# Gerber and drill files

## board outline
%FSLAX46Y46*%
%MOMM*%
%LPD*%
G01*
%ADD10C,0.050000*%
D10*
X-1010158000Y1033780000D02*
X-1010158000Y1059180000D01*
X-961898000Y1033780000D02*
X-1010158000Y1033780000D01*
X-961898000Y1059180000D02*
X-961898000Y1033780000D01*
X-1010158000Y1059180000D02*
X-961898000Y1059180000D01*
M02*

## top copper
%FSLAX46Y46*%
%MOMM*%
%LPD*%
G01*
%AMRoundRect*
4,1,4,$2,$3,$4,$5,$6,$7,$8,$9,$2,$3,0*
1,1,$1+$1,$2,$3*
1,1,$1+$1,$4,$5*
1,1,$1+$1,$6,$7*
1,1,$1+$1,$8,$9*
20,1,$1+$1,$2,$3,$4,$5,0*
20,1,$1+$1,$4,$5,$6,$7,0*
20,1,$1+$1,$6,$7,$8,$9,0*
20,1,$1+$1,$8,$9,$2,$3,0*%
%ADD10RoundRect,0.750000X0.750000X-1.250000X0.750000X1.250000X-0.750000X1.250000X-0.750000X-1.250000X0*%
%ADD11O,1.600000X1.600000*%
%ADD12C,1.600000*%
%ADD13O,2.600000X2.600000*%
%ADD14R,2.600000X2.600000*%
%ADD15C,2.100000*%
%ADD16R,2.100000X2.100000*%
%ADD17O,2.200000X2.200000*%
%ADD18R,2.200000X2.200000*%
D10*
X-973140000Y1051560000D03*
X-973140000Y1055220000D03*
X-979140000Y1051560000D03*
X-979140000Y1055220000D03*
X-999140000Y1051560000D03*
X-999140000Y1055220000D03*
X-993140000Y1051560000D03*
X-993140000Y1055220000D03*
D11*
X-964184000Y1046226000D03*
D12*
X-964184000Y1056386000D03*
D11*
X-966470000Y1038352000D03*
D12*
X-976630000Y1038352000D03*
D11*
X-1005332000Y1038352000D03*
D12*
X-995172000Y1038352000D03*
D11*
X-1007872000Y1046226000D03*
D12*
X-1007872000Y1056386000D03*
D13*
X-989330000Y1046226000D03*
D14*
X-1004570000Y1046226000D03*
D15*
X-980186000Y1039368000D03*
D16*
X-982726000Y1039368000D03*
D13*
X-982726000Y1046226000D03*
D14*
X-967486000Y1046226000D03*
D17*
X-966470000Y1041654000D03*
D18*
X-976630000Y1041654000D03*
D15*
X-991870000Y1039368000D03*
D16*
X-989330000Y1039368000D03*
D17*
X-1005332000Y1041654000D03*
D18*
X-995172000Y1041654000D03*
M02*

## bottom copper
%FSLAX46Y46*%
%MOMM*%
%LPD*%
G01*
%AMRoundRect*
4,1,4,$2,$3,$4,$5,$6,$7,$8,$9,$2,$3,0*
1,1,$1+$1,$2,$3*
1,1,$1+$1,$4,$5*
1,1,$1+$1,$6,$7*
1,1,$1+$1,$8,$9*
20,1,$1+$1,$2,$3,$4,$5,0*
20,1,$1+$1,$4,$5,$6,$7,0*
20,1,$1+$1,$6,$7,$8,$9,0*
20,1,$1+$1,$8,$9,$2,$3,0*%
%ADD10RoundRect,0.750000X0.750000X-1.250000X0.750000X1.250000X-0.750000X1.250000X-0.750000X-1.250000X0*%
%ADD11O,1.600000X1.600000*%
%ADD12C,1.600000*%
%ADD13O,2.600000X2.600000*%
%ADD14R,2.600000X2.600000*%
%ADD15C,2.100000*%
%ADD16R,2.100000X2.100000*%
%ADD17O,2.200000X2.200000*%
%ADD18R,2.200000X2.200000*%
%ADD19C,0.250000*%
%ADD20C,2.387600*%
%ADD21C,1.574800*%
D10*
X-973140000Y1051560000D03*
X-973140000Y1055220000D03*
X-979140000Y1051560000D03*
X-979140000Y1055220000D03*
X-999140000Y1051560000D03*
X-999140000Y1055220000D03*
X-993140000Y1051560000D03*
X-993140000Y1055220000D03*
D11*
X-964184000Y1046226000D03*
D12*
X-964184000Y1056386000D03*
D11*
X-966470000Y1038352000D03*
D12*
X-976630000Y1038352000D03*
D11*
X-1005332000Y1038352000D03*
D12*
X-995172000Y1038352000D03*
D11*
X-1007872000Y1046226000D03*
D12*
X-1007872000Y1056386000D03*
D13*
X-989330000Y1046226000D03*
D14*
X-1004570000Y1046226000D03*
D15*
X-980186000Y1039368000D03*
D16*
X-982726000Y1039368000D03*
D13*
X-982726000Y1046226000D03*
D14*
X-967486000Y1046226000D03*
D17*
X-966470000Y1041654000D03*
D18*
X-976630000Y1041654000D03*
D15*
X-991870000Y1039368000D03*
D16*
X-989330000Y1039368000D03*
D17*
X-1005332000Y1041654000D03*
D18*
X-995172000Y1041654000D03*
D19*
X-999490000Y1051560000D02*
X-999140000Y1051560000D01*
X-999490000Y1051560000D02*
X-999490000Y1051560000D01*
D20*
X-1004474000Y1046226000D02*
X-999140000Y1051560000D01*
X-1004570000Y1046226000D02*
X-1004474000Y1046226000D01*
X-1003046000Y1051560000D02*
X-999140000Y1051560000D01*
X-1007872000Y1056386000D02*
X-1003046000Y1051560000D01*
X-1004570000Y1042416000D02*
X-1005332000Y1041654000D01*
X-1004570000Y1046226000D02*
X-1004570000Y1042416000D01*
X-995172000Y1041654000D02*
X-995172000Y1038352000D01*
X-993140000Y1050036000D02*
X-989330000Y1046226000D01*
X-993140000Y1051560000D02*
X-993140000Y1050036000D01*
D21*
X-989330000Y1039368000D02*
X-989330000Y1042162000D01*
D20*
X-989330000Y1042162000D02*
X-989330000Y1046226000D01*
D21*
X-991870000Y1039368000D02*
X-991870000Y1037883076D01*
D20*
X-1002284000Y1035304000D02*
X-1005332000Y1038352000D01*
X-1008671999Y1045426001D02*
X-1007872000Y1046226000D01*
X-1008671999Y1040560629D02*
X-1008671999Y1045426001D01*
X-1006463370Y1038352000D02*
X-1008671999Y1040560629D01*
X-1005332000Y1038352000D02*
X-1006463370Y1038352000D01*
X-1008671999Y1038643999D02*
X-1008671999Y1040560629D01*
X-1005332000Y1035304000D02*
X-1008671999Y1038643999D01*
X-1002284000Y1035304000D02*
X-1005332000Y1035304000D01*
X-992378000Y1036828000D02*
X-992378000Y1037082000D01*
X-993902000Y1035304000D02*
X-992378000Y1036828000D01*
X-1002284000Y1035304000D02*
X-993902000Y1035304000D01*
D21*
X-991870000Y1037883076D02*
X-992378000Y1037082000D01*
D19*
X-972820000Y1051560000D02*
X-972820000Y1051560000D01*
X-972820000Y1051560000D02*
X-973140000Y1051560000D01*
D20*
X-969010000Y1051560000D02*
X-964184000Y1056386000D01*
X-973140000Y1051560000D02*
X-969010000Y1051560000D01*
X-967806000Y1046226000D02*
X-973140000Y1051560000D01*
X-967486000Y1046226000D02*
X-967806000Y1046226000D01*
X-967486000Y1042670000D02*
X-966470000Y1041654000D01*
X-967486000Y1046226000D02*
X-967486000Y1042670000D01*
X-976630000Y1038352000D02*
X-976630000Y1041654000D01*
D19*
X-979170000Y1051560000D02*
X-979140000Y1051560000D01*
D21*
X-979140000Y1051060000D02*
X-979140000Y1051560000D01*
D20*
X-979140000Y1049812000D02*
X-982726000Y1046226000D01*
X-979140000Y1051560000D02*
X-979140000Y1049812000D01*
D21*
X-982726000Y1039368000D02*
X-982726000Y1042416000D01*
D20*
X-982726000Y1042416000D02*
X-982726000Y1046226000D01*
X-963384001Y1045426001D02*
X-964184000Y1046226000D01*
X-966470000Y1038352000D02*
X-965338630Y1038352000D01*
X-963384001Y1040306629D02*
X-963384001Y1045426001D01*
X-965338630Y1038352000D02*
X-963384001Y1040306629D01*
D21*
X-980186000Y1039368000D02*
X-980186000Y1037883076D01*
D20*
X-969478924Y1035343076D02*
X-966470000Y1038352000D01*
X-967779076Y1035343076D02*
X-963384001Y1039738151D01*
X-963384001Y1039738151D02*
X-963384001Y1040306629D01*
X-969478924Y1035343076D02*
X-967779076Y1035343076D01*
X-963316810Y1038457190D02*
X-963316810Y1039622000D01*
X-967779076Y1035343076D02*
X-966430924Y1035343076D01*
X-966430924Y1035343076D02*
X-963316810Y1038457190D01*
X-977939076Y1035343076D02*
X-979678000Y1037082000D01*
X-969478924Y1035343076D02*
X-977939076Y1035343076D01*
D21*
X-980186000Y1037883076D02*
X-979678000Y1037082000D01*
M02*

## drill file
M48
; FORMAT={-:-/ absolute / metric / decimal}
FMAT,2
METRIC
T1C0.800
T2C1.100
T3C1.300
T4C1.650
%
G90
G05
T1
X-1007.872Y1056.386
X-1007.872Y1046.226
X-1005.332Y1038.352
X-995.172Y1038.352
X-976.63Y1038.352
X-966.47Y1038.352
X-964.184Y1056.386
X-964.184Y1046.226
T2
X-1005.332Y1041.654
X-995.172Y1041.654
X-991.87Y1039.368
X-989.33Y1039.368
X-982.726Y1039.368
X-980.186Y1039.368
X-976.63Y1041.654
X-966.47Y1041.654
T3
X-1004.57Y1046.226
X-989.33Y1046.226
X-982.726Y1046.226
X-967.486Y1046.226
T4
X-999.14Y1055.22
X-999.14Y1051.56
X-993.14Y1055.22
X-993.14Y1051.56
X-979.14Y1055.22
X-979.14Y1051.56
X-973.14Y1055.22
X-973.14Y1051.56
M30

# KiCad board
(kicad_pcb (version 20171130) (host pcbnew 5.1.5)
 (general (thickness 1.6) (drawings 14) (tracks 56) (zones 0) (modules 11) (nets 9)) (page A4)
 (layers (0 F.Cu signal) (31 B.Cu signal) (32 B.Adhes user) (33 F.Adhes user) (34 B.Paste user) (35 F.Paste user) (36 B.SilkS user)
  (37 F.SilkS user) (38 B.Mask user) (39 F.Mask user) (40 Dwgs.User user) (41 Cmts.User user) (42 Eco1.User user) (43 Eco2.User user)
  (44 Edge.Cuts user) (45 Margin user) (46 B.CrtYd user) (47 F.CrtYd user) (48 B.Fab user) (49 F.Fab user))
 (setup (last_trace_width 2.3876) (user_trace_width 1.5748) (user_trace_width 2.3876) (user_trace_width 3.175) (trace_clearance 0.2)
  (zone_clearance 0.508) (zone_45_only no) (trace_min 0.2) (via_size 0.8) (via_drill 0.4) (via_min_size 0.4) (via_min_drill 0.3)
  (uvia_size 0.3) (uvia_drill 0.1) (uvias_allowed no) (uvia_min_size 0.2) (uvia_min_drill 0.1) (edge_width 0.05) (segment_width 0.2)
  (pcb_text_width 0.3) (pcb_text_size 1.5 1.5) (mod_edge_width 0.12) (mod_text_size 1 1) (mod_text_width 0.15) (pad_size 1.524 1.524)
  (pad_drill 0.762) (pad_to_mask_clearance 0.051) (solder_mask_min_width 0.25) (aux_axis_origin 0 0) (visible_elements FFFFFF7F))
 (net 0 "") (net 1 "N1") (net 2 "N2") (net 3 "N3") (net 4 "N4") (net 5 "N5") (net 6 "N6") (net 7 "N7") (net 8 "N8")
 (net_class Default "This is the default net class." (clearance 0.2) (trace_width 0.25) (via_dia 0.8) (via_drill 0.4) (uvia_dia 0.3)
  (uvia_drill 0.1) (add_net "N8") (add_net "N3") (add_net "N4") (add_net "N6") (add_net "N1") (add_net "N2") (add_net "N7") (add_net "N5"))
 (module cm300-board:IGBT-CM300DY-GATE (layer F.Cu) (at -1000.64 -1049.56)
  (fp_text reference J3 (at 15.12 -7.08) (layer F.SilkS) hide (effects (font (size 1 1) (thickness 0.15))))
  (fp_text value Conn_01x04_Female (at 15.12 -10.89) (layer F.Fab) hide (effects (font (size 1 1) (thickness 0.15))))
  (pad 4 thru_hole roundrect (at 27.5 -2 90) (size 4 3) (drill 1.65) (layers *.Cu *.Mask) (roundrect_rratio 0.25) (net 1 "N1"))
  (pad 4 thru_hole roundrect (at 27.5 -5.66 90) (size 4 3) (drill 1.65) (layers *.Cu *.Mask) (roundrect_rratio 0.25) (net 1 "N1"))
  (pad 3 thru_hole roundrect (at 21.5 -2 90) (size 4 3) (drill 1.65) (layers *.Cu *.Mask) (roundrect_rratio 0.25) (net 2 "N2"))
  (pad 3 thru_hole roundrect (at 21.5 -5.66 90) (size 4 3) (drill 1.65) (layers *.Cu *.Mask) (roundrect_rratio 0.25) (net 2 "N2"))
  (pad 1 thru_hole roundrect (at 1.5 -2 90) (size 4 3) (drill 1.65) (layers *.Cu *.Mask) (roundrect_rratio 0.25) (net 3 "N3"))
  (pad 1 thru_hole roundrect (at 1.5 -5.66 90) (size 4 3) (drill 1.65) (layers *.Cu *.Mask) (roundrect_rratio 0.25) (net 3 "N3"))
  (pad 2 thru_hole roundrect (at 7.5 -2 90) (size 4 3) (drill 1.65) (layers *.Cu *.Mask) (roundrect_rratio 0.25) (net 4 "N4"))
  (pad 2 thru_hole roundrect (at 7.5 -5.66 90) (size 4 3) (drill 1.65) (layers *.Cu *.Mask) (roundrect_rratio 0.25) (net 4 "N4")))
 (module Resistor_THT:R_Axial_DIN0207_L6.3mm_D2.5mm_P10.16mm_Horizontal (layer F.Cu) (at -964.184 -1056.386 270)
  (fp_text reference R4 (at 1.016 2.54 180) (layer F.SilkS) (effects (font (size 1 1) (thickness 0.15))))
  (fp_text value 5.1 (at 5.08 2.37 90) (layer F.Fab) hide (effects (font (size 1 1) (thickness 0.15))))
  (pad 2 thru_hole oval (at 10.16 0 270) (size 1.6 1.6) (drill 0.8) (layers *.Cu *.Mask) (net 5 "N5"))
  (pad 1 thru_hole circle (at 0 0 270) (size 1.6 1.6) (drill 0.8) (layers *.Cu *.Mask) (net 1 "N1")))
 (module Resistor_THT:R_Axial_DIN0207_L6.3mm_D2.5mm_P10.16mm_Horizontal (layer F.Cu) (at -976.63 -1038.352)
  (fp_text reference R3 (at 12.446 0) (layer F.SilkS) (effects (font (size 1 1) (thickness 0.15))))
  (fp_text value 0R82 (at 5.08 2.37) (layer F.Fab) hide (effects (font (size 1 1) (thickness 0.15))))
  (pad 2 thru_hole oval (at 10.16 0) (size 1.6 1.6) (drill 0.8) (layers *.Cu *.Mask) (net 5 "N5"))
  (pad 1 thru_hole circle (at 0 0) (size 1.6 1.6) (drill 0.8) (layers *.Cu *.Mask) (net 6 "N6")))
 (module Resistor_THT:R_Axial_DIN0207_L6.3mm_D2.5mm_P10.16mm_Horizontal (layer F.Cu) (at -995.172 -1038.352 180)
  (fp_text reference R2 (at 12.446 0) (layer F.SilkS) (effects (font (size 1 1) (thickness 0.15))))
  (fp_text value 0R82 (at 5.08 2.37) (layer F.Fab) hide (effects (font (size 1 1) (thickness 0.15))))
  (pad 2 thru_hole oval (at 10.16 0 180) (size 1.6 1.6) (drill 0.8) (layers *.Cu *.Mask) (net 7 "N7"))
  (pad 1 thru_hole circle (at 0 0 180) (size 1.6 1.6) (drill 0.8) (layers *.Cu *.Mask) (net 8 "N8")))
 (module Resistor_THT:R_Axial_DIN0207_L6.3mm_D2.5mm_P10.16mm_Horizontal (layer F.Cu) (at -1007.872 -1056.386 270)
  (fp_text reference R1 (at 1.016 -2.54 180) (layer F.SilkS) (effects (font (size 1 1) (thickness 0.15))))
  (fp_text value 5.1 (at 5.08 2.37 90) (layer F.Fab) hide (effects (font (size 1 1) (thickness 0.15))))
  (pad 2 thru_hole oval (at 10.16 0 270) (size 1.6 1.6) (drill 0.8) (layers *.Cu *.Mask) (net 7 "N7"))
  (pad 1 thru_hole circle (at 0 0 270) (size 1.6 1.6) (drill 0.8) (layers *.Cu *.Mask) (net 3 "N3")))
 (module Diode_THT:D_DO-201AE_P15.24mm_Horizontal (layer F.Cu) (at -1004.57 -1046.226)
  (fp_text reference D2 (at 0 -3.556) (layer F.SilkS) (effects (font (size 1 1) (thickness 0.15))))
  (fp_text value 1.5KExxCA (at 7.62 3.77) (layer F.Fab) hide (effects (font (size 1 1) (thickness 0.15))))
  (pad 2 thru_hole oval (at 15.24 0) (size 2.6 2.6) (drill 1.3) (layers *.Cu *.Mask) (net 4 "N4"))
  (pad 1 thru_hole rect (at 0 0) (size 2.6 2.6) (drill 1.3) (layers *.Cu *.Mask) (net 3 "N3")))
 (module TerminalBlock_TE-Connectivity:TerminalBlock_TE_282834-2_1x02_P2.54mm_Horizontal (layer F.Cu) (at -982.726 -1039.368)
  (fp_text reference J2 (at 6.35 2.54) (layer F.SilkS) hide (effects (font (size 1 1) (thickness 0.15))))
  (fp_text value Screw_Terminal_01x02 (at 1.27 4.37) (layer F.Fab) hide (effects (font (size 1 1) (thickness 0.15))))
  (pad 2 thru_hole circle (at 2.54 0) (size 2.1 2.1) (drill 1.1) (layers *.Cu *.Mask) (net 5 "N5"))
  (pad 1 thru_hole rect (at 0 0) (size 2.1 2.1) (drill 1.1) (layers *.Cu *.Mask) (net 2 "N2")))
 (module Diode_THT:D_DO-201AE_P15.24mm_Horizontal (layer F.Cu) (at -967.486 -1046.226 180)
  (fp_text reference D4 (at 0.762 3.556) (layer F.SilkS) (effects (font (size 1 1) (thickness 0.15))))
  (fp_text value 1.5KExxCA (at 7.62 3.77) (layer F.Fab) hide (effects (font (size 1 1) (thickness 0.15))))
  (pad 2 thru_hole oval (at 15.24 0 180) (size 2.6 2.6) (drill 1.3) (layers *.Cu *.Mask) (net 2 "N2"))
  (pad 1 thru_hole rect (at 0 0 180) (size 2.6 2.6) (drill 1.3) (layers *.Cu *.Mask) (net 1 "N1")))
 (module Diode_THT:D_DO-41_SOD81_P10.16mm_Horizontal (layer F.Cu) (at -976.63 -1041.654)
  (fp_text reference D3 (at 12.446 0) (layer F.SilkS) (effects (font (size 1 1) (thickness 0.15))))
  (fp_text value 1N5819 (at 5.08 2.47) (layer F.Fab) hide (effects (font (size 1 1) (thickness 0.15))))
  (pad 2 thru_hole oval (at 10.16 0) (size 2.2 2.2) (drill 1.1) (layers *.Cu *.Mask) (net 1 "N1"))
  (pad 1 thru_hole rect (at 0 0) (size 2.2 2.2) (drill 1.1) (layers *.Cu *.Mask) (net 6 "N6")))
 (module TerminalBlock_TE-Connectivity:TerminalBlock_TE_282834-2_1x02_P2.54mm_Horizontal (layer F.Cu) (at -989.33 -1039.368 180)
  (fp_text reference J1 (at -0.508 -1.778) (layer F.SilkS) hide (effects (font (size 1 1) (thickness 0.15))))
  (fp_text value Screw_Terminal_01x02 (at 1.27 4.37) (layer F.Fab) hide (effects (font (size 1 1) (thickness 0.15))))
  (pad 2 thru_hole circle (at 2.54 0 180) (size 2.1 2.1) (drill 1.1) (layers *.Cu *.Mask) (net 7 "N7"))
  (pad 1 thru_hole rect (at 0 0 180) (size 2.1 2.1) (drill 1.1) (layers *.Cu *.Mask) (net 4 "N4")))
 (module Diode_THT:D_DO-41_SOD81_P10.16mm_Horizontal (layer F.Cu) (at -995.172 -1041.654 180)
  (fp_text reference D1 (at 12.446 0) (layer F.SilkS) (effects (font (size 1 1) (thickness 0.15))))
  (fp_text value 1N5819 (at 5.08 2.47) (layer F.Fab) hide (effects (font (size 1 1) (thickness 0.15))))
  (pad 2 thru_hole oval (at 10.16 0 180) (size 2.2 2.2) (drill 1.1) (layers *.Cu *.Mask) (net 3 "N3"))
  (pad 1 thru_hole rect (at 0 0 180) (size 2.2 2.2) (drill 1.1) (layers *.Cu *.Mask) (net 8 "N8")))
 (gr_line (start -1010.158 -1033.78) (end -1010.158 -1059.18) (layer Edge.Cuts) (width 0.05))
 (gr_line (start -961.898 -1033.78) (end -1010.158 -1033.78) (layer Edge.Cuts) (width 0.05))
 (gr_line (start -961.898 -1059.18) (end -961.898 -1033.78) (layer Edge.Cuts) (width 0.05))
 (gr_line (start -1010.158 -1059.18) (end -961.898 -1059.18) (layer Edge.Cuts) (width 0.05))
 (segment (start -999.49 -1051.56) (end -999.14 -1051.56) (width 0.25) (layer B.Cu) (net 3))
 (segment (start -999.49 -1051.56) (end -999.49 -1051.56) (width 0.25) (layer B.Cu) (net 3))
 (segment (start -1004.474 -1046.226) (end -999.14 -1051.56) (width 2.3876) (layer B.Cu) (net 3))
 (segment (start -1004.57 -1046.226) (end -1004.474 -1046.226) (width 2.3876) (layer B.Cu) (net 3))
 (segment (start -1003.046 -1051.56) (end -999.14 -1051.56) (width 2.3876) (layer B.Cu) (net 3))
 (segment (start -1007.872 -1056.386) (end -1003.046 -1051.56) (width 2.3876) (layer B.Cu) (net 3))
 (segment (start -1004.57 -1042.416) (end -1005.332 -1041.654) (width 2.3876) (layer B.Cu) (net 3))
 (segment (start -1004.57 -1046.226) (end -1004.57 -1042.416) (width 2.3876) (layer B.Cu) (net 3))
 (segment (start -995.172 -1041.654) (end -995.172 -1038.352) (width 2.3876) (layer B.Cu) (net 8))
 (segment (start -993.14 -1050.036) (end -989.33 -1046.226) (width 2.3876) (layer B.Cu) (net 4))
 (segment (start -993.14 -1051.56) (end -993.14 -1050.036) (width 2.3876) (layer B.Cu) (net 4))
 (segment (start -989.33 -1039.368) (end -989.33 -1042.162) (width 1.5748) (layer B.Cu) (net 4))
 (segment (start -989.33 -1042.162) (end -989.33 -1046.226) (width 2.3876) (layer B.Cu) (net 4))
 (segment (start -991.87 -1039.368) (end -991.87 -1037.883076) (width 1.5748) (layer B.Cu) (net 7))
 (segment (start -1002.284 -1035.304) (end -1005.332 -1038.352) (width 2.3876) (layer B.Cu) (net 7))
 (segment (start -1008.671999 -1045.426001) (end -1007.872 -1046.226) (width 2.3876) (layer B.Cu) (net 7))
 (segment (start -1008.671999 -1040.560629) (end -1008.671999 -1045.426001) (width 2.3876) (layer B.Cu) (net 7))
 (segment (start -1006.46337 -1038.352) (end -1008.671999 -1040.560629) (width 2.3876) (layer B.Cu) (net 7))
 (segment (start -1005.332 -1038.352) (end -1006.46337 -1038.352) (width 2.3876) (layer B.Cu) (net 7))
 (segment (start -1008.671999 -1038.643999) (end -1008.671999 -1040.560629) (width 2.3876) (layer B.Cu) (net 7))
 (segment (start -1005.332 -1035.304) (end -1008.671999 -1038.643999) (width 2.3876) (layer B.Cu) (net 7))
 (segment (start -1002.284 -1035.304) (end -1005.332 -1035.304) (width 2.3876) (layer B.Cu) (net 7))
 (segment (start -992.378 -1036.828) (end -992.378 -1037.082) (width 2.3876) (layer B.Cu) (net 7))
 (segment (start -993.902 -1035.304) (end -992.378 -1036.828) (width 2.3876) (layer B.Cu) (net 7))
 (segment (start -1002.284 -1035.304) (end -993.902 -1035.304) (width 2.3876) (layer B.Cu) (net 7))
 (segment (start -991.87 -1037.883076) (end -992.378 -1037.082) (width 1.5748) (layer B.Cu) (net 7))
 (segment (start -972.82 -1051.56) (end -972.82 -1051.56) (width 0.25) (layer B.Cu) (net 1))
 (segment (start -972.82 -1051.56) (end -973.14 -1051.56) (width 0.25) (layer B.Cu) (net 1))
 (segment (start -969.01 -1051.56) (end -964.184 -1056.386) (width 2.3876) (layer B.Cu) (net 1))
 (segment (start -973.14 -1051.56) (end -969.01 -1051.56) (width 2.3876) (layer B.Cu) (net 1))
 (segment (start -967.806 -1046.226) (end -973.14 -1051.56) (width 2.3876) (layer B.Cu) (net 1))
 (segment (start -967.486 -1046.226) (end -967.806 -1046.226) (width 2.3876) (layer B.Cu) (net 1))
 (segment (start -967.486 -1042.67) (end -966.47 -1041.654) (width 2.3876) (layer B.Cu) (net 1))
 (segment (start -967.486 -1046.226) (end -967.486 -1042.67) (width 2.3876) (layer B.Cu) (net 1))
 (segment (start -976.63 -1038.352) (end -976.63 -1041.654) (width 2.3876) (layer B.Cu) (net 6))
 (segment (start -979.17 -1051.56) (end -979.14 -1051.56) (width 0.25) (layer B.Cu) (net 2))
 (segment (start -979.14 -1051.06) (end -979.14 -1051.56) (width 1.5748) (layer B.Cu) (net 2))
 (segment (start -979.14 -1049.812) (end -982.726 -1046.226) (width 2.3876) (layer B.Cu) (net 2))
 (segment (start -979.14 -1051.56) (end -979.14 -1049.812) (width 2.3876) (layer B.Cu) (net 2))
 (segment (start -982.726 -1039.368) (end -982.726 -1042.416) (width 1.5748) (layer B.Cu) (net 2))
 (segment (start -982.726 -1042.416) (end -982.726 -1046.226) (width 2.3876) (layer B.Cu) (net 2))
 (segment (start -963.384001 -1045.426001) (end -964.184 -1046.226) (width 2.3876) (layer B.Cu) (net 5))
 (segment (start -966.47 -1038.352) (end -965.33863 -1038.352) (width 2.3876) (layer B.Cu) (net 5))
 (segment (start -963.384001 -1040.306629) (end -963.384001 -1045.426001) (width 2.3876) (layer B.Cu) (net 5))
 (segment (start -965.33863 -1038.352) (end -963.384001 -1040.306629) (width 2.3876) (layer B.Cu) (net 5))
 (segment (start -980.186 -1039.368) (end -980.186 -1037.883076) (width 1.5748) (layer B.Cu) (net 5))
 (segment (start -969.478924 -1035.343076) (end -966.47 -1038.352) (width 2.3876) (layer B.Cu) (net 5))
 (segment (start -967.779076 -1035.343076) (end -963.384001 -1039.738151) (width 2.3876) (layer B.Cu) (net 5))
 (segment (start -963.384001 -1039.738151) (end -963.384001 -1040.306629) (width 2.3876) (layer B.Cu) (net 5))
 (segment (start -969.478924 -1035.343076) (end -967.779076 -1035.343076) (width 2.3876) (layer B.Cu) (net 5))
 (segment (start -963.31681 -1038.45719) (end -963.31681 -1039.622) (width 2.3876) (layer B.Cu) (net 5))
 (segment (start -967.779076 -1035.343076) (end -966.430924 -1035.343076) (width 2.3876) (layer B.Cu) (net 5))
 (segment (start -966.430924 -1035.343076) (end -963.31681 -1038.45719) (width 2.3876) (layer B.Cu) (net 5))
 (segment (start -977.939076 -1035.343076) (end -979.678 -1037.082) (width 2.3876) (layer B.Cu) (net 5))
 (segment (start -969.478924 -1035.343076) (end -977.939076 -1035.343076) (width 2.3876) (layer B.Cu) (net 5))
 (segment (start -980.186 -1037.883076) (end -979.678 -1037.082) (width 1.5748) (layer B.Cu) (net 5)))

